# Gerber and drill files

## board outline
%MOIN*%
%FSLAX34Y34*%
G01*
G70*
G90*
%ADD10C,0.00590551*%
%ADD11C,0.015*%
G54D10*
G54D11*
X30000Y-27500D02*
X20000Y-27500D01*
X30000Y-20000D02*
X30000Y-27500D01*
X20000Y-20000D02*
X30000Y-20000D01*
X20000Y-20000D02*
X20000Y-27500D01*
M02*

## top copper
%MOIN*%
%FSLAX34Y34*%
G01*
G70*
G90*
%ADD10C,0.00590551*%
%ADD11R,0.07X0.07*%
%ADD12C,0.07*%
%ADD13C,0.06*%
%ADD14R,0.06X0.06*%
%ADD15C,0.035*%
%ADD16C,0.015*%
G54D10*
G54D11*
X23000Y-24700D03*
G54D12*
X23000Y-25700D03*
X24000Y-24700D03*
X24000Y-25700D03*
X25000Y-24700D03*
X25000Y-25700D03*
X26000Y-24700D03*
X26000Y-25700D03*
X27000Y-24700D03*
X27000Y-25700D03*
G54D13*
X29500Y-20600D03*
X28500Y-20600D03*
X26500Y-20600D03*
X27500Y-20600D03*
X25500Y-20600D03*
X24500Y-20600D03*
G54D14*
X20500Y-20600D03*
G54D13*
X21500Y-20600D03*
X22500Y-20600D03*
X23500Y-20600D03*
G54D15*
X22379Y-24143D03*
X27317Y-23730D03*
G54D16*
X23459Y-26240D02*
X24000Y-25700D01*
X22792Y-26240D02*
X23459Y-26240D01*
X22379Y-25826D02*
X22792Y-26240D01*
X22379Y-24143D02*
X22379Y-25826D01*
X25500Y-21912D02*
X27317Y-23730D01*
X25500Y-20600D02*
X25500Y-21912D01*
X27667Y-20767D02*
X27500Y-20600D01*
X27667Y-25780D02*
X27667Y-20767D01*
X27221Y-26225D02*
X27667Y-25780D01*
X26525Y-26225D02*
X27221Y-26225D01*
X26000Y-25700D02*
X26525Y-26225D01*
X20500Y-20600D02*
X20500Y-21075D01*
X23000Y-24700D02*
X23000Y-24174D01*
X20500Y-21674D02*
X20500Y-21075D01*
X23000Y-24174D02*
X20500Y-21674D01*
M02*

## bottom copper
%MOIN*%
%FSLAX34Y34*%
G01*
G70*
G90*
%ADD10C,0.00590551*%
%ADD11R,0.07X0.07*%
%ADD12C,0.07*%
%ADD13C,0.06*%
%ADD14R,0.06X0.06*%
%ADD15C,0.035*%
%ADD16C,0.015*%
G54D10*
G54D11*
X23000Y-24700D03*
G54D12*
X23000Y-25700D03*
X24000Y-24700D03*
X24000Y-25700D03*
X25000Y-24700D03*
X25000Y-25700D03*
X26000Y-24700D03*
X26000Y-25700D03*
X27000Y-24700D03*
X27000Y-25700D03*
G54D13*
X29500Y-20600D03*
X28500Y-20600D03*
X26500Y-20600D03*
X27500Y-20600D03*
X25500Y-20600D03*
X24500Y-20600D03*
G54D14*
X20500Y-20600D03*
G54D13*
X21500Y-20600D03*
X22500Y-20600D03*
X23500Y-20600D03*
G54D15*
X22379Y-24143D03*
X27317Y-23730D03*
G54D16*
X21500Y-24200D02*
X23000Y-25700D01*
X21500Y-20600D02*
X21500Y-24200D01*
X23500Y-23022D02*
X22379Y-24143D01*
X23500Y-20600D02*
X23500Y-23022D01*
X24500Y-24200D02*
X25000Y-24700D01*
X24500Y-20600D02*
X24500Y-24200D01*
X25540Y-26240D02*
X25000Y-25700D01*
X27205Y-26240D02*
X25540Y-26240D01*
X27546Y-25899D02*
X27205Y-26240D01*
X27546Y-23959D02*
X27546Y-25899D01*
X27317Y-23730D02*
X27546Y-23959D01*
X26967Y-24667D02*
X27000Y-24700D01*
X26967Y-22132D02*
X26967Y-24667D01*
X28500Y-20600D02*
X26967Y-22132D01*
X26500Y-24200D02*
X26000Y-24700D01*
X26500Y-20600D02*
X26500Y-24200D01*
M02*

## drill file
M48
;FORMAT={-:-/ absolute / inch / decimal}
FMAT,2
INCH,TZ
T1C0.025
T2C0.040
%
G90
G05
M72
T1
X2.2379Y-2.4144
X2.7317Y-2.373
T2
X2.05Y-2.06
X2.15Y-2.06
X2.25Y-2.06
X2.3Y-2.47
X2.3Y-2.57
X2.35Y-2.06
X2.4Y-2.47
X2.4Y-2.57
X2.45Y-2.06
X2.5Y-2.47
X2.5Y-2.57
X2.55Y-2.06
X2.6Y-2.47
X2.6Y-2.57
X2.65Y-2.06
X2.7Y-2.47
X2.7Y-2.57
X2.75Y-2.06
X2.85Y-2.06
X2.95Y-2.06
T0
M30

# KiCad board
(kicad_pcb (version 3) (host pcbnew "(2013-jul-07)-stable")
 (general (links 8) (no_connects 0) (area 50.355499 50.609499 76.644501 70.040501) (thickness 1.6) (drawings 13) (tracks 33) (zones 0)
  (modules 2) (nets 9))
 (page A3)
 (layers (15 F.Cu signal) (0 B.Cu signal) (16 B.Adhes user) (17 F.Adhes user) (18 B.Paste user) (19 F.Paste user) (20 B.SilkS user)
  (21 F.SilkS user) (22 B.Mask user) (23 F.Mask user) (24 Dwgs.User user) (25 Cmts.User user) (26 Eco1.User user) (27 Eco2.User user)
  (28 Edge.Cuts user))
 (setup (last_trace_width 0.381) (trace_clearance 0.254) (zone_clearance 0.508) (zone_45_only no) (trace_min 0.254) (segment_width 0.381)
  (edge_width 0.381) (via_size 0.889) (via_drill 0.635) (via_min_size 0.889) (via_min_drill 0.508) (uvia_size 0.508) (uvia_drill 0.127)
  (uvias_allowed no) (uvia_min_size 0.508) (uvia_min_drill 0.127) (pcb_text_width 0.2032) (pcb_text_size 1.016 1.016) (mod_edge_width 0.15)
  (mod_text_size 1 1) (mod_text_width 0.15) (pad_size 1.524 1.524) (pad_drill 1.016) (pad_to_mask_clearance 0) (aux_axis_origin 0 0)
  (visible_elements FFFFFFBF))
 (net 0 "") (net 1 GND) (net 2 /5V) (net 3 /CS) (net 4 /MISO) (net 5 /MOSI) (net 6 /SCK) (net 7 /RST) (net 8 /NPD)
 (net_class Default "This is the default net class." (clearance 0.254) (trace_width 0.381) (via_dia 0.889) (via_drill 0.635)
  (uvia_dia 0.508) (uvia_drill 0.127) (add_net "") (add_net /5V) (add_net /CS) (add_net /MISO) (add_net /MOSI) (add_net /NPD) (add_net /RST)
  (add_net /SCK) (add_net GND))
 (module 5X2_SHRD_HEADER (layer B.Cu) (at 63.5 64.008)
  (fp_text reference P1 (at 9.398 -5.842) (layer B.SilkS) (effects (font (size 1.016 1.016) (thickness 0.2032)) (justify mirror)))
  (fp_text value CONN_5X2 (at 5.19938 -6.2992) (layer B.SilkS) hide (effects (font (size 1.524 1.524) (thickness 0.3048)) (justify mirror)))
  (pad 1 thru_hole rect (at -5.08 -1.27) (size 1.778 1.778) (drill 1.016) (layers *.Cu *.Mask B.SilkS) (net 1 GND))
  (pad 2 thru_hole circle (at -5.08 1.27) (size 1.778 1.778) (drill 1.016) (layers *.Cu *.Mask B.SilkS) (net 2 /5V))
  (pad 3 thru_hole circle (at -2.54 -1.27) (size 1.778 1.778) (drill 1.016) (layers *.Cu *.Mask B.SilkS))
  (pad 4 thru_hole circle (at -2.54 1.27) (size 1.778 1.778) (drill 1.016) (layers *.Cu *.Mask B.SilkS) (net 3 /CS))
  (pad 5 thru_hole circle (at 0 -1.27) (size 1.778 1.778) (drill 1.016) (layers *.Cu *.Mask B.SilkS) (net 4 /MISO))
  (pad 6 thru_hole circle (at 0 1.27) (size 1.778 1.778) (drill 1.016) (layers *.Cu *.Mask B.SilkS) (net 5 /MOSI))
  (pad 7 thru_hole circle (at 2.54 -1.27) (size 1.778 1.778) (drill 1.016) (layers *.Cu *.Mask B.SilkS) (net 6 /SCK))
  (pad 8 thru_hole circle (at 2.54 1.27) (size 1.778 1.778) (drill 1.016) (layers *.Cu *.Mask B.SilkS) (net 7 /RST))
  (pad 9 thru_hole circle (at 5.08 -1.27) (size 1.778 1.778) (drill 1.016) (layers *.Cu *.Mask B.SilkS) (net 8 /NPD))
  (pad 10 thru_hole circle (at 5.08 1.27) (size 1.778 1.778) (drill 1.016) (layers *.Cu *.Mask B.SilkS)))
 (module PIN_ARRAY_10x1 (layer F.Cu) (at 63.5 52.324)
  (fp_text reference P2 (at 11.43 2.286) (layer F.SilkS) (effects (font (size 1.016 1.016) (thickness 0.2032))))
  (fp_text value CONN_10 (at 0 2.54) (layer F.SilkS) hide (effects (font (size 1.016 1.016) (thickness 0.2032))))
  (pad 10 thru_hole circle (at 11.43 0) (size 1.524 1.524) (drill 1.016) (layers *.Cu *.Mask F.SilkS))
  (pad 9 thru_hole circle (at 8.89 0) (size 1.524 1.524) (drill 1.016) (layers *.Cu *.Mask F.SilkS) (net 8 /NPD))
  (pad 7 thru_hole circle (at 3.81 0) (size 1.524 1.524) (drill 1.016) (layers *.Cu *.Mask F.SilkS) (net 6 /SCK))
  (pad 8 thru_hole circle (at 6.35 0) (size 1.524 1.524) (drill 1.016) (layers *.Cu *.Mask F.SilkS) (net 7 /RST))
  (pad 6 thru_hole circle (at 1.27 0) (size 1.524 1.524) (drill 1.016) (layers *.Cu *.Mask F.SilkS) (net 5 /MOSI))
  (pad 5 thru_hole circle (at -1.27 0) (size 1.524 1.524) (drill 1.016) (layers *.Cu *.Mask F.SilkS) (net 4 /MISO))
  (pad 1 thru_hole rect (at -11.43 0) (size 1.524 1.524) (drill 1.016) (layers *.Cu *.Mask F.SilkS) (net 1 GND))
  (pad 2 thru_hole circle (at -8.89 0) (size 1.524 1.524) (drill 1.016) (layers *.Cu *.Mask F.SilkS) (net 2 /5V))
  (pad 3 thru_hole circle (at -6.35 0) (size 1.524 1.524) (drill 1.016) (layers *.Cu *.Mask F.SilkS))
  (pad 4 thru_hole circle (at -3.81 0) (size 1.524 1.524) (drill 1.016) (layers *.Cu *.Mask F.SilkS) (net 3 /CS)))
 (gr_line (start 76.2 69.85) (end 50.8 69.85) (angle 90) (layer Edge.Cuts) (width 0.381))
 (gr_line (start 76.2 50.8) (end 76.2 69.85) (angle 90) (layer Edge.Cuts) (width 0.381))
 (gr_line (start 50.8 50.8) (end 76.2 50.8) (angle 90) (layer Edge.Cuts) (width 0.381))
 (gr_line (start 50.8 50.8) (end 50.8 69.85) (angle 90) (layer Edge.Cuts) (width 0.381))
 (segment (start 54.61 61.468) (end 58.42 65.278) (width 0.381) (layer B.Cu) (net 2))
 (segment (start 54.61 52.324) (end 54.61 61.468) (width 0.381) (layer B.Cu) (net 2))
 (via (at 56.8434 61.325) (size 0.889) (layers F.Cu B.Cu) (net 3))
 (segment (start 59.69 58.4784) (end 56.8434 61.325) (width 0.381) (layer B.Cu) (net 3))
 (segment (start 59.69 52.324) (end 59.69 58.4784) (width 0.381) (layer B.Cu) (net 3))
 (segment (start 59.5874 66.6506) (end 60.96 65.278) (width 0.381) (layer F.Cu) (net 3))
 (segment (start 57.8941 66.6506) (end 59.5874 66.6506) (width 0.381) (layer F.Cu) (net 3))
 (segment (start 56.8434 65.5999) (end 57.8941 66.6506) (width 0.381) (layer F.Cu) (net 3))
 (segment (start 56.8434 61.325) (end 56.8434 65.5999) (width 0.381) (layer F.Cu) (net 3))
 (segment (start 62.23 61.468) (end 63.5 62.738) (width 0.381) (layer B.Cu) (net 4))
 (segment (start 62.23 52.324) (end 62.23 61.468) (width 0.381) (layer B.Cu) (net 4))
 (via (at 69.386 60.2749) (size 0.889) (layers F.Cu B.Cu) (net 5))
 (segment (start 64.77 55.6589) (end 69.386 60.2749) (width 0.381) (layer F.Cu) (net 5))
 (segment (start 64.77 52.324) (end 64.77 55.6589) (width 0.381) (layer F.Cu) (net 5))
 (segment (start 64.8725 66.6505) (end 63.5 65.278) (width 0.381) (layer B.Cu) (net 5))
 (segment (start 69.1023 66.6505) (end 64.8725 66.6505) (width 0.381) (layer B.Cu) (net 5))
 (segment (start 69.9676 65.7852) (end 69.1023 66.6505) (width 0.381) (layer B.Cu) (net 5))
 (segment (start 69.9676 60.8565) (end 69.9676 65.7852) (width 0.381) (layer B.Cu) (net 5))
 (segment (start 69.386 60.2749) (end 69.9676 60.8565) (width 0.381) (layer B.Cu) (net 5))
 (segment (start 68.4967 62.6547) (end 68.58 62.738) (width 0.381) (layer B.Cu) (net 8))
 (segment (start 68.4967 56.2173) (end 68.4967 62.6547) (width 0.381) (layer B.Cu) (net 8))
 (segment (start 72.39 52.324) (end 68.4967 56.2173) (width 0.381) (layer B.Cu) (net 8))
 (segment (start 70.2753 52.7493) (end 69.85 52.324) (width 0.381) (layer F.Cu) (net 7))
 (segment (start 70.2753 65.4812) (end 70.2753 52.7493) (width 0.381) (layer F.Cu) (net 7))
 (segment (start 69.1429 66.6136) (end 70.2753 65.4812) (width 0.381) (layer F.Cu) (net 7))
 (segment (start 67.3756 66.6136) (end 69.1429 66.6136) (width 0.381) (layer F.Cu) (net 7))
 (segment (start 66.04 65.278) (end 67.3756 66.6136) (width 0.381) (layer F.Cu) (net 7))
 (segment (start 67.31 61.468) (end 66.04 62.738) (width 0.381) (layer B.Cu) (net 6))
 (segment (start 67.31 52.324) (end 67.31 61.468) (width 0.381) (layer B.Cu) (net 6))
 (segment (start 52.07 52.324) (end 52.07 53.5308) (width 0.381) (layer F.Cu) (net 1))
 (segment (start 58.42 62.738) (end 58.42 61.4042) (width 0.381) (layer F.Cu) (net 1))
 (segment (start 52.07 55.0542) (end 52.07 53.5308) (width 0.381) (layer F.Cu) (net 1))
 (segment (start 58.42 61.4042) (end 52.07 55.0542) (width 0.381) (layer F.Cu) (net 1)))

